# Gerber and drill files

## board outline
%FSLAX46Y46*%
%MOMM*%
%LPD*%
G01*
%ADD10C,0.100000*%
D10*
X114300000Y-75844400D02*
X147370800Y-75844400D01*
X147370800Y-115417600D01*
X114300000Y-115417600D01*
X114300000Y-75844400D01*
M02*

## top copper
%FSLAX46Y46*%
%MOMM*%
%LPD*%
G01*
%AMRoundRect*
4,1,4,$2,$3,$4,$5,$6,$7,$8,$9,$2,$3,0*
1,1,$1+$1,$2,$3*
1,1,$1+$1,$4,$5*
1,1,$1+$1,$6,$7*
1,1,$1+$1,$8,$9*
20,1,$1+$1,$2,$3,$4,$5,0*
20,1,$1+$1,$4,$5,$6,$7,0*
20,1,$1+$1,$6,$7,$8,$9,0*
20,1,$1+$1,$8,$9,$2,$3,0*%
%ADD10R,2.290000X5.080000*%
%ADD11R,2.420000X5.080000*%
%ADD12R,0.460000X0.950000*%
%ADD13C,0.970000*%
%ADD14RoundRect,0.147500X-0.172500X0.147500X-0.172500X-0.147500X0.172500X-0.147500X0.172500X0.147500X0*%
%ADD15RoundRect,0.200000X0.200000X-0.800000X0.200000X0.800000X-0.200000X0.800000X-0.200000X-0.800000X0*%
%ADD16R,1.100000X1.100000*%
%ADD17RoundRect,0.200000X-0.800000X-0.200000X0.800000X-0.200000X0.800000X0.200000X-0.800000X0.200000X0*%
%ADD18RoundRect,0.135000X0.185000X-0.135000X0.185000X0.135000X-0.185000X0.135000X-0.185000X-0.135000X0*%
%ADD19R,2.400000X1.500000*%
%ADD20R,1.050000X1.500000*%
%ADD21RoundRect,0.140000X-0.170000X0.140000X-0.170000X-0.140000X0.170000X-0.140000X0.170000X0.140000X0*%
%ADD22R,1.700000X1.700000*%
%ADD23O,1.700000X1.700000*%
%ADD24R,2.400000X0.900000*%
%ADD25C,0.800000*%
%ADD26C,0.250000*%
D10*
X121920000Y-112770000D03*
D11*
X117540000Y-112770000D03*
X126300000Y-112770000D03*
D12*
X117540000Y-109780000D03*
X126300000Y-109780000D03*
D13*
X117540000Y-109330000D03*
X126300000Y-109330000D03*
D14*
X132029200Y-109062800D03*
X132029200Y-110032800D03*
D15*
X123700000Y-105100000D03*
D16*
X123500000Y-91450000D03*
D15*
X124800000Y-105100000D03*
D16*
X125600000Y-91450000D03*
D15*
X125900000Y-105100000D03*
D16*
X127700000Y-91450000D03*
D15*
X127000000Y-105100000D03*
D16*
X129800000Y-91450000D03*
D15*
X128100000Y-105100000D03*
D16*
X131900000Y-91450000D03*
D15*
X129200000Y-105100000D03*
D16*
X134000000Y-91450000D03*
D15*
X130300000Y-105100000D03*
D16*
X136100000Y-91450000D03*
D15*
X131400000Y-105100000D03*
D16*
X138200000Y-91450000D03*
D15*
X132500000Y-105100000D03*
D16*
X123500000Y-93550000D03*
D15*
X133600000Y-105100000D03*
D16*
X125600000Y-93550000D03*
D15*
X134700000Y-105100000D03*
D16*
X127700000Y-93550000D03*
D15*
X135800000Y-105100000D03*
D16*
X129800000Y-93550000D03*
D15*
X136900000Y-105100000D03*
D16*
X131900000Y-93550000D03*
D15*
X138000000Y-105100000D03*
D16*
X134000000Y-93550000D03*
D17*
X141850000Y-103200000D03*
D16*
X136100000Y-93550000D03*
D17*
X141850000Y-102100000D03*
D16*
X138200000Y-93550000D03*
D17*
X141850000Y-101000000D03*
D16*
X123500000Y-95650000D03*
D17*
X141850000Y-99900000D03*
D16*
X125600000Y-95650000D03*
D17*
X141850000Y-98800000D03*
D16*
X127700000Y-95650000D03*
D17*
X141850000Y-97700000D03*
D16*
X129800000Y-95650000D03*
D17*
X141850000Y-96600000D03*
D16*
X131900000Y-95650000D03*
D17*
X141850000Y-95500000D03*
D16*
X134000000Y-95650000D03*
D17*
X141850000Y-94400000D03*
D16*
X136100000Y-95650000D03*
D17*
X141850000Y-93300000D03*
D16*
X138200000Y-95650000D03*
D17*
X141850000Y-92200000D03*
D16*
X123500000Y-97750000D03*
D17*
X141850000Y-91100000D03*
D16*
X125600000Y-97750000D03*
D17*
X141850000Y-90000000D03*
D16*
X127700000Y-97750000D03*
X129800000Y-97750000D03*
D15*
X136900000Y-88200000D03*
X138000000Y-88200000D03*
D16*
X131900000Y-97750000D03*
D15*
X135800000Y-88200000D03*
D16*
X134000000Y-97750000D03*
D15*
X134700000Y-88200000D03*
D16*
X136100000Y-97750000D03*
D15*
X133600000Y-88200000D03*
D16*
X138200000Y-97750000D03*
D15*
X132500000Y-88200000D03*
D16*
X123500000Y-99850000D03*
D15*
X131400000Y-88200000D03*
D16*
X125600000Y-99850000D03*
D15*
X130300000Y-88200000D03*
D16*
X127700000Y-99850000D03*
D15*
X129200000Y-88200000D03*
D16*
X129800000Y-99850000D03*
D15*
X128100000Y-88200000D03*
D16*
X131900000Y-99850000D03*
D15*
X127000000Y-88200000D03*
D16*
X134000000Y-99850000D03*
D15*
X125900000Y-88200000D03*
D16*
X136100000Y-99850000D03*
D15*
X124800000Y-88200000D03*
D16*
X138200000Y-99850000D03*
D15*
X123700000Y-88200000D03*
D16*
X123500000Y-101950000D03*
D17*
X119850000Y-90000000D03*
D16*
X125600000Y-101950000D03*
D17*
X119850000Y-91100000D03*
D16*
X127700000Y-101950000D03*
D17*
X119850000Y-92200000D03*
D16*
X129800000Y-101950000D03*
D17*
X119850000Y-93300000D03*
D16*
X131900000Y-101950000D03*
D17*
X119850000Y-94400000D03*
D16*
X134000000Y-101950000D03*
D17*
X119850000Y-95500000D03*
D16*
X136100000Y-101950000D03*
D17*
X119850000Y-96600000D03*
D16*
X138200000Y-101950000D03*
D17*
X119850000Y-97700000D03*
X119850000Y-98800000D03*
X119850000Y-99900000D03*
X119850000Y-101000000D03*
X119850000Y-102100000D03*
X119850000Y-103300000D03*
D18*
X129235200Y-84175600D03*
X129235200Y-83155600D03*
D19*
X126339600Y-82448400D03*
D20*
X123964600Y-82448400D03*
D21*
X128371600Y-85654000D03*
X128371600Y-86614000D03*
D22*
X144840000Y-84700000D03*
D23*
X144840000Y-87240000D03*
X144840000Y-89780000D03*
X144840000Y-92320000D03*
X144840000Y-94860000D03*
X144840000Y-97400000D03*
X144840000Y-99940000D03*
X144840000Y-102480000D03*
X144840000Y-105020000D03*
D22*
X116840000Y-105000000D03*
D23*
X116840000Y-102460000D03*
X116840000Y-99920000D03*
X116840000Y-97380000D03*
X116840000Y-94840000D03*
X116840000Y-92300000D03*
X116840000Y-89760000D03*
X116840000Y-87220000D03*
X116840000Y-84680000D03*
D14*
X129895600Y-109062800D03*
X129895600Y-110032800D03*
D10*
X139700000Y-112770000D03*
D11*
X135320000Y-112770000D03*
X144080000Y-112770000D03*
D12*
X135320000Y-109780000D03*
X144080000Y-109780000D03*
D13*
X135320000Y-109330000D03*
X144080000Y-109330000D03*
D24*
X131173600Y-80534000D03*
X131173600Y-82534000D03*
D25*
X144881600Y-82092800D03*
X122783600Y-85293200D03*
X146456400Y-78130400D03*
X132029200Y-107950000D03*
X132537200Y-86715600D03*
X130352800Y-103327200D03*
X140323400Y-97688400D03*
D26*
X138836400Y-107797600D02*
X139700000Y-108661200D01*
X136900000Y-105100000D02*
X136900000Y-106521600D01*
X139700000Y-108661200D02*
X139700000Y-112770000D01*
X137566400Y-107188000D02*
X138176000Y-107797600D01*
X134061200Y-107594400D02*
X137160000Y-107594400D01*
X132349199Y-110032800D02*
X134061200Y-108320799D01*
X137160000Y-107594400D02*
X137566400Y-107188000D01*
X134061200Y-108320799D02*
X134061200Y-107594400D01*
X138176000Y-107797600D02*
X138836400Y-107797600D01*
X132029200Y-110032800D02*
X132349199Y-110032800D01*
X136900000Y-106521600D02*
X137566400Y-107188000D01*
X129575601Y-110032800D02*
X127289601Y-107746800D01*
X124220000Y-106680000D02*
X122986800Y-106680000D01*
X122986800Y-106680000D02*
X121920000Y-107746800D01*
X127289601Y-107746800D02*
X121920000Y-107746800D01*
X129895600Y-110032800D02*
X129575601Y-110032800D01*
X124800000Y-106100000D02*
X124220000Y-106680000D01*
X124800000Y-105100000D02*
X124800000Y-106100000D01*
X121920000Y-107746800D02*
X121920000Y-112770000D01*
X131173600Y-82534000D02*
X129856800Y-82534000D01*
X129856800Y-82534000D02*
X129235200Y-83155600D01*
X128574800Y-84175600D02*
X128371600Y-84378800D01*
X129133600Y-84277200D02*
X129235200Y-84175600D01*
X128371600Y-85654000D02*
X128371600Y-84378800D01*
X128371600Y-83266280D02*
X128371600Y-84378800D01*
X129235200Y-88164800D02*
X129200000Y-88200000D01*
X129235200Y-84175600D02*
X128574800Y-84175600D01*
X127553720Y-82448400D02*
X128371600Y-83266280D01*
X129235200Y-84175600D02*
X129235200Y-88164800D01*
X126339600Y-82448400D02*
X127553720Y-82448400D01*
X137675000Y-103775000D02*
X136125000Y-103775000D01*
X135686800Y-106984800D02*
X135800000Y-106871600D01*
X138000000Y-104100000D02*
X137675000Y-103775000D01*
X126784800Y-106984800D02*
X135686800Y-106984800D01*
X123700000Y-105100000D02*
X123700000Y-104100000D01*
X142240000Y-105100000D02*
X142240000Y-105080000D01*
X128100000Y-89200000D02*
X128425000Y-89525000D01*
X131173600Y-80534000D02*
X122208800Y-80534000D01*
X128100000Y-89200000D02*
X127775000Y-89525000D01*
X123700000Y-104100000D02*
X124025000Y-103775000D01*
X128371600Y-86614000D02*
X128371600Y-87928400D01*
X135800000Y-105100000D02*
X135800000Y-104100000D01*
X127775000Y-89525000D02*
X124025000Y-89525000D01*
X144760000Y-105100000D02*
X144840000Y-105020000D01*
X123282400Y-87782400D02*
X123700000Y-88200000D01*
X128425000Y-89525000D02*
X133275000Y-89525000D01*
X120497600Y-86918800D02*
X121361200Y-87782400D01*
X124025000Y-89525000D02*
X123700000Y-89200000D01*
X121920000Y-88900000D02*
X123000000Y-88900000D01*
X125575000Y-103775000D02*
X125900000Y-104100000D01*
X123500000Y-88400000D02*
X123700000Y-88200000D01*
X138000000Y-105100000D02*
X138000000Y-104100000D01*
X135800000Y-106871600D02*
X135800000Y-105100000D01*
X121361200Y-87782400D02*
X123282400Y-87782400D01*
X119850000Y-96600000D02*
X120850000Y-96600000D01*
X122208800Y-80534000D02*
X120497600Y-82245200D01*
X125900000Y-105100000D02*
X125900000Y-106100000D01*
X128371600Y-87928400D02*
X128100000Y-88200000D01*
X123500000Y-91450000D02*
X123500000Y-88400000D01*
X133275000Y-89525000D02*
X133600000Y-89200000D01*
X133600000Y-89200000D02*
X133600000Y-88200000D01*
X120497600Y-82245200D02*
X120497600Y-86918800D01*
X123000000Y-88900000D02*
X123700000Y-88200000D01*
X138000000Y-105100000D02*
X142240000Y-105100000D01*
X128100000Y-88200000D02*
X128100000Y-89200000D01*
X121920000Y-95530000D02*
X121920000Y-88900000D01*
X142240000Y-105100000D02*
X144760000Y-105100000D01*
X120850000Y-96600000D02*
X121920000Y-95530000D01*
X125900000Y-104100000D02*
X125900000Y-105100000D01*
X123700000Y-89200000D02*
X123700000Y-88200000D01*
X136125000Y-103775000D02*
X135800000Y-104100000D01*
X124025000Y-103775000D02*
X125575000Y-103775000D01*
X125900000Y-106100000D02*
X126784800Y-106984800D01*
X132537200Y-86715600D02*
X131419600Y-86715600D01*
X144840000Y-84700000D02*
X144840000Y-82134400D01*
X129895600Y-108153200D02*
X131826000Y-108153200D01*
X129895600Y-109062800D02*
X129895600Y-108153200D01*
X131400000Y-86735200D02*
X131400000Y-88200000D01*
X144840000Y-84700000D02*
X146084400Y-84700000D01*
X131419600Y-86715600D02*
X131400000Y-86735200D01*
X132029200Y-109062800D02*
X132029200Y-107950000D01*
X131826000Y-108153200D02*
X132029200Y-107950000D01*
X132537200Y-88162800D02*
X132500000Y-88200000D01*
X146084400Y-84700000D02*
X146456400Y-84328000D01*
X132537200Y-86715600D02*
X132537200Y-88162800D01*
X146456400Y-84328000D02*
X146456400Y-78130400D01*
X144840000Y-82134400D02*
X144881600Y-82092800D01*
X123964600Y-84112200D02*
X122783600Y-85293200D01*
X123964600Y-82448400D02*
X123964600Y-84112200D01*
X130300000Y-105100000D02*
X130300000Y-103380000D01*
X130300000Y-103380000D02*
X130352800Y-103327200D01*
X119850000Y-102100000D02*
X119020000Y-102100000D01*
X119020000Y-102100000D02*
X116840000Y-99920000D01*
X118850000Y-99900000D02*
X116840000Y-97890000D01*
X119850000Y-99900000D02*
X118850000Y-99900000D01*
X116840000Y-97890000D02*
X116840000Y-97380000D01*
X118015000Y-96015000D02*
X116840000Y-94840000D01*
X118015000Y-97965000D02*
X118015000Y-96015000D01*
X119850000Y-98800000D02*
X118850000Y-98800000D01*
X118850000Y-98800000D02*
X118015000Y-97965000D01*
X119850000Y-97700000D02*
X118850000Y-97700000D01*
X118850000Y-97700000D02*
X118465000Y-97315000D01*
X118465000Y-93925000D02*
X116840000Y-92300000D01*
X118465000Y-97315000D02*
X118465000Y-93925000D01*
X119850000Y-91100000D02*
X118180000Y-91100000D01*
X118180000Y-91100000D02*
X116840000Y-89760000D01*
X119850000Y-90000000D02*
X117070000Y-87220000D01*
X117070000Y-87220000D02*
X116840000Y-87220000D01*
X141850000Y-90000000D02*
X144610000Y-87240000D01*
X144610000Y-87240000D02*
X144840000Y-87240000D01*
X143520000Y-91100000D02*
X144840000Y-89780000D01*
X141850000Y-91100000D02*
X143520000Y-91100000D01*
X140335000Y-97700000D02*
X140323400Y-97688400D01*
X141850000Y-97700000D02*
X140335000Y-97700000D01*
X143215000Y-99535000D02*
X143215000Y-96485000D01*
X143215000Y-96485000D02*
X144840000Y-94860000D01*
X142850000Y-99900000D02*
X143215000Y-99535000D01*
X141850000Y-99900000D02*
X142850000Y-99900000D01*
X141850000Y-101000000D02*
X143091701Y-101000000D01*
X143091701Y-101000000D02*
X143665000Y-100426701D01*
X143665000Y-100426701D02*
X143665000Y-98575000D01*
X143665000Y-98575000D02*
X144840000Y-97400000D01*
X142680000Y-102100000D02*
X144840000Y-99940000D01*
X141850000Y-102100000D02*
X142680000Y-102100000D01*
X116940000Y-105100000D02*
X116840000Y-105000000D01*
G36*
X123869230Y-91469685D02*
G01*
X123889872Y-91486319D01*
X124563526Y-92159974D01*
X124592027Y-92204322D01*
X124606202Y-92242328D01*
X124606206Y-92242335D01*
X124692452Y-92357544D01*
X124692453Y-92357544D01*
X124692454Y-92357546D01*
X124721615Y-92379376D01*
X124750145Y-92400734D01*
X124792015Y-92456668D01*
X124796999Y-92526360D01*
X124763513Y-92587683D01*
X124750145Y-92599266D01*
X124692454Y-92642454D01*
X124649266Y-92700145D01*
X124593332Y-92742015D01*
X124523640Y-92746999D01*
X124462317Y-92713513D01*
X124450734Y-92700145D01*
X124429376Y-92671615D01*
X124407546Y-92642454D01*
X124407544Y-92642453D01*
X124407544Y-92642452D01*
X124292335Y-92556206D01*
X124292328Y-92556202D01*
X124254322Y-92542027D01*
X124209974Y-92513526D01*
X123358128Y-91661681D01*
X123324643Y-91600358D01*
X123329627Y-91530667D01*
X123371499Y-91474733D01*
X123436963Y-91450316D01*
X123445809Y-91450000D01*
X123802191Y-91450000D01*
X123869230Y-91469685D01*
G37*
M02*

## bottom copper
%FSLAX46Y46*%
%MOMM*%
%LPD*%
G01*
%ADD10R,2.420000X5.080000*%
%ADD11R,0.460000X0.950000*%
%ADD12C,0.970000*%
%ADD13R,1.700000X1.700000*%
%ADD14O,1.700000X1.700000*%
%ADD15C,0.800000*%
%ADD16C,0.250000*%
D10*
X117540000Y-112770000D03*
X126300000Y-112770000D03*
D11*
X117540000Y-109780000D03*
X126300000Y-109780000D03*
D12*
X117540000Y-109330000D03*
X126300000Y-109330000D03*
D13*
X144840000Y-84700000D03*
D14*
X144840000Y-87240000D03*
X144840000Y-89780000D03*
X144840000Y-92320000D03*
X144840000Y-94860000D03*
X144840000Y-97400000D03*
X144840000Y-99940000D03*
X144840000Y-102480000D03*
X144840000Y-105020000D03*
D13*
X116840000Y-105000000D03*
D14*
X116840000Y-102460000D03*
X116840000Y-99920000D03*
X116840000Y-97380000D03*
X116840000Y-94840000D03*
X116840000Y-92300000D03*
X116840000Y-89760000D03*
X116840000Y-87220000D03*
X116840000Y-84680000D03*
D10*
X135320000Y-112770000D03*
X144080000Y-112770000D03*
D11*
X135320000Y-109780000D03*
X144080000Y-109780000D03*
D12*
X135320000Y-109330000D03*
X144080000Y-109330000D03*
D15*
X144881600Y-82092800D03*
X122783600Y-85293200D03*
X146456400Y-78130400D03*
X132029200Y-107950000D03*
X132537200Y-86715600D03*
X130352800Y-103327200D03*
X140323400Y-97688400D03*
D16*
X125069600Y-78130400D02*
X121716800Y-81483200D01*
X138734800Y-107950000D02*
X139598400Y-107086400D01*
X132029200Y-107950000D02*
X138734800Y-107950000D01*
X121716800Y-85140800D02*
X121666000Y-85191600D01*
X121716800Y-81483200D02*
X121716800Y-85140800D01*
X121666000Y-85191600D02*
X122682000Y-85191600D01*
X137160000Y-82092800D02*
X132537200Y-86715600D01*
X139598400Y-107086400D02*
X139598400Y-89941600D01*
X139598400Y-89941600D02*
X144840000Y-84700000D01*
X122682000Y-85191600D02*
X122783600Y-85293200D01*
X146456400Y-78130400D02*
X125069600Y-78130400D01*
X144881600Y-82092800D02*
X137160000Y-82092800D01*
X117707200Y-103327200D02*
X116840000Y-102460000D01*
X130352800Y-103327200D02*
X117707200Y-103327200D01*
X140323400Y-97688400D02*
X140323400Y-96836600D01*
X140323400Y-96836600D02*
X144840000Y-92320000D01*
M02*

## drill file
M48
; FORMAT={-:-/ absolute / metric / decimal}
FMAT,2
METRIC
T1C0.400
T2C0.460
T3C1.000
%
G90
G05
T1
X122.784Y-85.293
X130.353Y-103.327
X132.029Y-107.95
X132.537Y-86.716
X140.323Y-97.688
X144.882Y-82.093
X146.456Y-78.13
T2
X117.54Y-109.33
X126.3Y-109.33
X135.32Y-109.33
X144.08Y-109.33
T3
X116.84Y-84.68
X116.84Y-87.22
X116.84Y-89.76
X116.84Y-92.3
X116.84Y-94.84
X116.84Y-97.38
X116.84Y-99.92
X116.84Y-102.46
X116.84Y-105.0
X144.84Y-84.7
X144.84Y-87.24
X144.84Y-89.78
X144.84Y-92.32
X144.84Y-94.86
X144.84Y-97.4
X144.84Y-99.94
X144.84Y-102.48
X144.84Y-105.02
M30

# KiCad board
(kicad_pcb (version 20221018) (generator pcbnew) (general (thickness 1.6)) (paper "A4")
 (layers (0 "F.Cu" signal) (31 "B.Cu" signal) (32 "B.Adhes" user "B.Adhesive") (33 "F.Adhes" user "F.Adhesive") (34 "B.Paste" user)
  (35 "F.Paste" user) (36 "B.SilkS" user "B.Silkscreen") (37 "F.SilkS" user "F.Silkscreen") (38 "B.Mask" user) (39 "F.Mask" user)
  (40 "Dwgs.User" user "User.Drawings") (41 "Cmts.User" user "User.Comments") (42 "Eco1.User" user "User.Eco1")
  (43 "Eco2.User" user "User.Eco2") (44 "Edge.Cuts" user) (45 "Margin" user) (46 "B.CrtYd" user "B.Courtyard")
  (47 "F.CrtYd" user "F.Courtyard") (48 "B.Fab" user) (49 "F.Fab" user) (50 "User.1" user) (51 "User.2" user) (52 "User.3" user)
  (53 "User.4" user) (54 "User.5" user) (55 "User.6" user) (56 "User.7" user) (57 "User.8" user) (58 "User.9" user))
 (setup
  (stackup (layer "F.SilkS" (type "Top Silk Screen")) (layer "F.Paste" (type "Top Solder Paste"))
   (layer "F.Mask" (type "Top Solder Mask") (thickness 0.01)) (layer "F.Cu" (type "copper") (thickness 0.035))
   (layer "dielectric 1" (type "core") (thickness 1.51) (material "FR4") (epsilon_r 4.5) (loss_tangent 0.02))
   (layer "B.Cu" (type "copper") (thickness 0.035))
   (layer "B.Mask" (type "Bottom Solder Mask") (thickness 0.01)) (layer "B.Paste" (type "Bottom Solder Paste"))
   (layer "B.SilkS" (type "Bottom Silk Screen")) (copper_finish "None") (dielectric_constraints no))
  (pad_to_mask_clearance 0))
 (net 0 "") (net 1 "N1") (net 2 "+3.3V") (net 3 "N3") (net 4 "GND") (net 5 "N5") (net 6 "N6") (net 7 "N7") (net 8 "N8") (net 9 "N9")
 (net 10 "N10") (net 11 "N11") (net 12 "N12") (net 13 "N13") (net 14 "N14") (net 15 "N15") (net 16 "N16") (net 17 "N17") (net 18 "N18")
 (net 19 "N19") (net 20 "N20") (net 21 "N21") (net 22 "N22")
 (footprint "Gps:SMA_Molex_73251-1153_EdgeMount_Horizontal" (layer "F.Cu") (at 121.92 111.05 90)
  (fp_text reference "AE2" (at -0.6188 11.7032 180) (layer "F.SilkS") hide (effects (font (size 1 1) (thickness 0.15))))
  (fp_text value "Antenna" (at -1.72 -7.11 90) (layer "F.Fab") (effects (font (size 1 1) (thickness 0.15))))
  (pad "1" smd rect (at -1.72 0 90) (size 5.08 2.29) (layers "F.Cu" "F.Paste" "F.Mask") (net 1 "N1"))
  (pad "2" smd rect (at -1.72 -4.38 90) (size 5.08 2.42) (layers "F.Cu" "F.Paste" "F.Mask"))
  (pad "2" smd rect (at -1.72 -4.38 90) (size 5.08 2.42) (layers "B.Cu" "B.Paste" "B.Mask"))
  (pad "2" smd rect (at -1.72 4.38 90) (size 5.08 2.42) (layers "F.Cu" "F.Paste" "F.Mask"))
  (pad "2" smd rect (at -1.72 4.38 90) (size 5.08 2.42) (layers "B.Cu" "B.Paste" "B.Mask"))
  (pad "2" smd rect (at 1.27 -4.38 90) (size 0.95 0.46) (layers "F.Cu"))
  (pad "2" smd rect (at 1.27 -4.38 90) (size 0.95 0.46) (layers "B.Cu"))
  (pad "2" smd rect (at 1.27 4.38 90) (size 0.95 0.46) (layers "F.Cu"))
  (pad "2" smd rect (at 1.27 4.38 90) (size 0.95 0.46) (layers "B.Cu"))
  (pad "2" thru_hole circle (at 1.72 -4.38 90) (size 0.97 0.97) (drill 0.46) (layers "*.Cu"))
  (pad "2" thru_hole circle (at 1.72 4.38 90) (size 0.97 0.97) (drill 0.46) (layers "*.Cu")))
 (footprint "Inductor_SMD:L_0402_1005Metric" (layer "F.Cu") (at 132.0292 109.5478 -90)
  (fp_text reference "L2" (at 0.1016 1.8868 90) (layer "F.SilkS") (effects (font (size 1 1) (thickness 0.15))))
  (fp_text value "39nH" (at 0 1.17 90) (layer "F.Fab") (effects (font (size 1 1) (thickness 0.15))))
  (pad "1" smd roundrect (at -0.485 0 270) (size 0.59 0.64) (layers "F.Cu" "F.Paste" "F.Mask") (roundrect_rratio 0.25) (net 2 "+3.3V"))
  (pad "2" smd roundrect (at 0.485 0 270) (size 0.59 0.64) (layers "F.Cu" "F.Paste" "F.Mask") (roundrect_rratio 0.25) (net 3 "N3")))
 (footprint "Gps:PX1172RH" (layer "F.Cu") (at 119.85 90)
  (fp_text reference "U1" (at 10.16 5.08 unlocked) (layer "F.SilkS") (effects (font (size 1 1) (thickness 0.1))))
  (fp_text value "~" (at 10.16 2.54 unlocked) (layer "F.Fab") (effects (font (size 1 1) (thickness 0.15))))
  (pad "1" smd roundrect (at 3.85 15.1 90) (size 2 0.8) (layers "F.Cu" "F.Paste" "F.Mask") (roundrect_rratio 0.25) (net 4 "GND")
   (thermal_bridge_angle 45))
  (pad "1$" smd rect (at 3.65 1.45) (size 1.1 1.1) (layers "F.Cu" "F.Paste" "F.Mask") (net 4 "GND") (thermal_bridge_angle 45))
  (pad "2" smd roundrect (at 4.95 15.1 90) (size 2 0.8) (layers "F.Cu" "F.Paste" "F.Mask") (roundrect_rratio 0.25) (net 1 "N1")
   (thermal_bridge_angle 45))
  (pad "2$" smd rect (at 5.75 1.45) (size 1.1 1.1) (layers "F.Cu" "F.Paste" "F.Mask") (thermal_bridge_angle 45))
  (pad "3" smd roundrect (at 6.05 15.1 90) (size 2 0.8) (layers "F.Cu" "F.Paste" "F.Mask") (roundrect_rratio 0.25) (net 4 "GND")
   (thermal_bridge_angle 45))
  (pad "3$" smd rect (at 7.85 1.45) (size 1.1 1.1) (layers "F.Cu" "F.Paste" "F.Mask") (thermal_bridge_angle 45))
  (pad "4" smd roundrect (at 7.15 15.1 90) (size 2 0.8) (layers "F.Cu" "F.Paste" "F.Mask") (roundrect_rratio 0.25) (thermal_bridge_angle 45))
  (pad "4$" smd rect (at 9.95 1.45) (size 1.1 1.1) (layers "F.Cu" "F.Paste" "F.Mask") (thermal_bridge_angle 45))
  (pad "5" smd roundrect (at 8.25 15.1 90) (size 2 0.8) (layers "F.Cu" "F.Paste" "F.Mask") (roundrect_rratio 0.25) (thermal_bridge_angle 45))
  (pad "5$" smd rect (at 12.05 1.45) (size 1.1 1.1) (layers "F.Cu" "F.Paste" "F.Mask") (thermal_bridge_angle 45))
  (pad "6" smd roundrect (at 9.35 15.1 90) (size 2 0.8) (layers "F.Cu" "F.Paste" "F.Mask") (roundrect_rratio 0.25) (thermal_bridge_angle 45))
  (pad "6$" smd rect (at 14.15 1.45) (size 1.1 1.1) (layers "F.Cu" "F.Paste" "F.Mask") (thermal_bridge_angle 45))
  (pad "7" smd roundrect (at 10.45 15.1 90) (size 2 0.8) (layers "F.Cu" "F.Paste" "F.Mask") (roundrect_rratio 0.25) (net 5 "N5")
   (thermal_bridge_angle 45))
  (pad "7$" smd rect (at 16.25 1.45) (size 1.1 1.1) (layers "F.Cu" "F.Paste" "F.Mask") (thermal_bridge_angle 45))
  (pad "8" smd roundrect (at 11.55 15.1 90) (size 2 0.8) (layers "F.Cu" "F.Paste" "F.Mask") (roundrect_rratio 0.25)
   (thermal_bridge_angle 45))
  (pad "8$" smd rect (at 18.35 1.45) (size 1.1 1.1) (layers "F.Cu" "F.Paste" "F.Mask") (thermal_bridge_angle 45))
  (pad "9" smd roundrect (at 12.65 15.1 90) (size 2 0.8) (layers "F.Cu" "F.Paste" "F.Mask") (roundrect_rratio 0.25)
   (thermal_bridge_angle 45))
  (pad "9$" smd rect (at 3.65 3.55) (size 1.1 1.1) (layers "F.Cu" "F.Paste" "F.Mask") (thermal_bridge_angle 45))
  (pad "10" smd roundrect (at 13.75 15.1 90) (size 2 0.8) (layers "F.Cu" "F.Paste" "F.Mask") (roundrect_rratio 0.25)
   (thermal_bridge_angle 45))
  (pad "10$" smd rect (at 5.75 3.55) (size 1.1 1.1) (layers "F.Cu" "F.Paste" "F.Mask") (thermal_bridge_angle 45))
  (pad "11" smd roundrect (at 14.85 15.1 90) (size 2 0.8) (layers "F.Cu" "F.Paste" "F.Mask") (roundrect_rratio 0.25)
   (thermal_bridge_angle 45))
  (pad "11$" smd rect (at 7.85 3.55) (size 1.1 1.1) (layers "F.Cu" "F.Paste" "F.Mask") (thermal_bridge_angle 45))
  (pad "12" smd roundrect (at 15.95 15.1 90) (size 2 0.8) (layers "F.Cu" "F.Paste" "F.Mask") (roundrect_rratio 0.25) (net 4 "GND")
   (thermal_bridge_angle 45))
  (pad "12$" smd rect (at 9.95 3.55) (size 1.1 1.1) (layers "F.Cu" "F.Paste" "F.Mask") (thermal_bridge_angle 45))
  (pad "13" smd roundrect (at 17.05 15.1 90) (size 2 0.8) (layers "F.Cu" "F.Paste" "F.Mask") (roundrect_rratio 0.25) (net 3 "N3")
   (thermal_bridge_angle 45))
  (pad "13$" smd rect (at 12.05 3.55) (size 1.1 1.1) (layers "F.Cu" "F.Paste" "F.Mask") (thermal_bridge_angle 45))
  (pad "14" smd roundrect (at 18.15 15.1 90) (size 2 0.8) (layers "F.Cu" "F.Paste" "F.Mask") (roundrect_rratio 0.25) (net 4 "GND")
   (thermal_bridge_angle 45))
  (pad "14$" smd rect (at 14.15 3.55) (size 1.1 1.1) (layers "F.Cu" "F.Paste" "F.Mask") (thermal_bridge_angle 45))
  (pad "15" smd roundrect (at 22 13.2) (size 2 0.8) (layers "F.Cu" "F.Paste" "F.Mask") (roundrect_rratio 0.25) (thermal_bridge_angle 45))
  (pad "15$" smd rect (at 16.25 3.55) (size 1.1 1.1) (layers "F.Cu" "F.Paste" "F.Mask") (thermal_bridge_angle 45))
  (pad "16" smd roundrect (at 22 12.1) (size 2 0.8) (layers "F.Cu" "F.Paste" "F.Mask") (roundrect_rratio 0.25) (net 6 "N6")
   (thermal_bridge_angle 45))
  (pad "16$" smd rect (at 18.35 3.55) (size 1.1 1.1) (layers "F.Cu" "F.Paste" "F.Mask") (thermal_bridge_angle 45))
  (pad "17" smd roundrect (at 22 11) (size 2 0.8) (layers "F.Cu" "F.Paste" "F.Mask") (roundrect_rratio 0.25) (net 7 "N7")
   (thermal_bridge_angle 45))
  (pad "17$" smd rect (at 3.65 5.65) (size 1.1 1.1) (layers "F.Cu" "F.Paste" "F.Mask") (thermal_bridge_angle 45))
  (pad "18" smd roundrect (at 22 9.9) (size 2 0.8) (layers "F.Cu" "F.Paste" "F.Mask") (roundrect_rratio 0.25) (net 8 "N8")
   (thermal_bridge_angle 45))
  (pad "18$" smd rect (at 5.75 5.65) (size 1.1 1.1) (layers "F.Cu" "F.Paste" "F.Mask") (thermal_bridge_angle 45))
  (pad "19" smd roundrect (at 22 8.8) (size 2 0.8) (layers "F.Cu" "F.Paste" "F.Mask") (roundrect_rratio 0.25) (thermal_bridge_angle 45))
  (pad "19$" smd rect (at 7.85 5.65) (size 1.1 1.1) (layers "F.Cu" "F.Paste" "F.Mask") (thermal_bridge_angle 45))
  (pad "20" smd roundrect (at 22 7.7) (size 2 0.8) (layers "F.Cu" "F.Paste" "F.Mask") (roundrect_rratio 0.25) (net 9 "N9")
   (thermal_bridge_angle 45))
  (pad "20$" smd rect (at 9.95 5.65) (size 1.1 1.1) (layers "F.Cu" "F.Paste" "F.Mask") (thermal_bridge_angle 45))
  (pad "21" smd roundrect (at 22 6.6) (size 2 0.8) (layers "F.Cu" "F.Paste" "F.Mask") (roundrect_rratio 0.25) (thermal_bridge_angle 45))
  (pad "21$" smd rect (at 12.05 5.65) (size 1.1 1.1) (layers "F.Cu" "F.Paste" "F.Mask") (thermal_bridge_angle 45))
  (pad "22" smd roundrect (at 22 5.5) (size 2 0.8) (layers "F.Cu" "F.Paste" "F.Mask") (roundrect_rratio 0.25) (thermal_bridge_angle 45))
  (pad "22$" smd rect (at 14.15 5.65) (size 1.1 1.1) (layers "F.Cu" "F.Paste" "F.Mask") (thermal_bridge_angle 45))
  (pad "23" smd roundrect (at 22 4.4) (size 2 0.8) (layers "F.Cu" "F.Paste" "F.Mask") (roundrect_rratio 0.25) (thermal_bridge_angle 45))
  (pad "23$" smd rect (at 16.25 5.65) (size 1.1 1.1) (layers "F.Cu" "F.Paste" "F.Mask") (thermal_bridge_angle 45))
  (pad "24" smd roundrect (at 22 3.3) (size 2 0.8) (layers "F.Cu" "F.Paste" "F.Mask") (roundrect_rratio 0.25) (thermal_bridge_angle 45))
  (pad "24$" smd rect (at 18.35 5.65) (size 1.1 1.1) (layers "F.Cu" "F.Paste" "F.Mask") (thermal_bridge_angle 45))
  (pad "25" smd roundrect (at 22 2.2) (size 2 0.8) (layers "F.Cu" "F.Mask") (roundrect_rratio 0.25) (thermal_bridge_angle 45))
  (pad "25$" smd rect (at 3.65 7.75) (size 1.1 1.1) (layers "F.Cu" "F.Paste" "F.Mask") (thermal_bridge_angle 45))
  (pad "26" smd roundrect (at 22 1.1) (size 2 0.8) (layers "F.Cu" "F.Paste" "F.Mask") (roundrect_rratio 0.25) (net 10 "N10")
   (thermal_bridge_angle 45))
  (pad "26$" smd rect (at 5.75 7.75) (size 1.1 1.1) (layers "F.Cu" "F.Paste" "F.Mask") (thermal_bridge_angle 45))
  (pad "27" smd roundrect (at 22 0) (size 2 0.8) (layers "F.Cu" "F.Paste" "F.Mask") (roundrect_rratio 0.25) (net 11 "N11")
   (thermal_bridge_angle 45))
  (pad "27$" smd rect (at 7.85 7.75) (size 1.1 1.1) (layers "F.Cu" "F.Paste" "F.Mask") (thermal_bridge_angle 45))
  (pad "28$" smd rect (at 9.95 7.75) (size 1.1 1.1) (layers "F.Cu" "F.Paste" "F.Mask") (thermal_bridge_angle 45))
  (pad "29" smd roundrect (at 17.05 -1.8 90) (size 2 0.8) (layers "F.Cu" "F.Paste" "F.Mask") (roundrect_rratio 0.25)
   (thermal_bridge_angle 45))
  (pad "29" smd roundrect (at 18.15 -1.8 90) (size 2 0.8) (layers "F.Cu" "F.Paste" "F.Mask") (roundrect_rratio 0.25)
   (thermal_bridge_angle 45))
  (pad "29$" smd rect (at 12.05 7.75) (size 1.1 1.1) (layers "F.Cu" "F.Paste" "F.Mask") (thermal_bridge_angle 45))
  (pad "30" smd roundrect (at 15.95 -1.8 90) (size 2 0.8) (layers "F.Cu" "F.Paste" "F.Mask") (roundrect_rratio 0.25)
   (thermal_bridge_angle 45))
  (pad "30$" smd rect (at 14.15 7.75) (size 1.1 1.1) (layers "F.Cu" "F.Paste" "F.Mask") (thermal_bridge_angle 45))
  (pad "31" smd roundrect (at 14.85 -1.8 90) (size 2 0.8) (layers "F.Cu" "F.Paste" "F.Mask") (roundrect_rratio 0.25)
   (thermal_bridge_angle 45))
  (pad "31$" smd rect (at 16.25 7.75) (size 1.1 1.1) (layers "F.Cu" "F.Paste" "F.Mask") (thermal_bridge_angle 45))
  (pad "32" smd roundrect (at 13.75 -1.8 90) (size 2 0.8) (layers "F.Cu" "F.Paste" "F.Mask") (roundrect_rratio 0.25) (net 4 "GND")
   (thermal_bridge_angle 45))
  (pad "32$" smd rect (at 18.35 7.75) (size 1.1 1.1) (layers "F.Cu" "F.Paste" "F.Mask") (thermal_bridge_angle 45))
  (pad "33" smd roundrect (at 12.65 -1.8 90) (size 2 0.8) (layers "F.Cu" "F.Paste" "F.Mask") (roundrect_rratio 0.25) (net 2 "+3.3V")
   (thermal_bridge_angle 45))
  (pad "33$" smd rect (at 3.65 9.85) (size 1.1 1.1) (layers "F.Cu" "F.Paste" "F.Mask") (thermal_bridge_angle 45))
  (pad "34" smd roundrect (at 11.55 -1.8 90) (size 2 0.8) (layers "F.Cu" "F.Paste" "F.Mask") (roundrect_rratio 0.25) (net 2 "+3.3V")
   (thermal_bridge_angle 45))
  (pad "34$" smd rect (at 5.75 9.85) (size 1.1 1.1) (layers "F.Cu" "F.Paste" "F.Mask") (thermal_bridge_angle 45))
  (pad "35" smd roundrect (at 10.45 -1.8 90) (size 2 0.8) (layers "F.Cu" "F.Paste" "F.Mask") (roundrect_rratio 0.25)
   (thermal_bridge_angle 45))
  (pad "35$" smd rect (at 7.85 9.85) (size 1.1 1.1) (layers "F.Cu" "F.Paste" "F.Mask") (thermal_bridge_angle 45))
  (pad "36" smd roundrect (at 9.35 -1.8 90) (size 2 0.8) (layers "F.Cu" "F.Paste" "F.Mask") (roundrect_rratio 0.25) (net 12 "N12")
   (thermal_bridge_angle 45))
  (pad "36$" smd rect (at 9.95 9.85) (size 1.1 1.1) (layers "F.Cu" "F.Paste" "F.Mask") (thermal_bridge_angle 45))
  (pad "37" smd roundrect (at 8.25 -1.8 90) (size 2 0.8) (layers "F.Cu" "F.Paste" "F.Mask") (roundrect_rratio 0.25) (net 4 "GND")
   (thermal_bridge_angle 45))
  (pad "37$" smd rect (at 12.05 9.85) (size 1.1 1.1) (layers "F.Cu" "F.Paste" "F.Mask") (thermal_bridge_angle 45))
  (pad "38" smd roundrect (at 7.15 -1.8 90) (size 2 0.8) (layers "F.Cu" "F.Paste" "F.Mask") (roundrect_rratio 0.25)
   (thermal_bridge_angle 45))
  (pad "38$" smd rect (at 14.15 9.85) (size 1.1 1.1) (layers "F.Cu" "F.Paste" "F.Mask") (thermal_bridge_angle 45))
  (pad "39" smd roundrect (at 6.05 -1.8 90) (size 2 0.8) (layers "F.Cu" "F.Paste" "F.Mask") (roundrect_rratio 0.25)
   (thermal_bridge_angle 45))
  (pad "39$" smd rect (at 16.25 9.85) (size 1.1 1.1) (layers "F.Cu" "F.Paste" "F.Mask") (thermal_bridge_angle 45))
  (pad "40" smd roundrect (at 4.95 -1.8 90) (size 2 0.8) (layers "F.Cu" "F.Paste" "F.Mask") (roundrect_rratio 0.25)
   (thermal_bridge_angle 45))
  (pad "40$" smd rect (at 18.35 9.85) (size 1.1 1.1) (layers "F.Cu" "F.Paste" "F.Mask") (thermal_bridge_angle 45))
  (pad "41" smd roundrect (at 3.85 -1.8 90) (size 2 0.8) (layers "F.Cu" "F.Paste" "F.Mask") (roundrect_rratio 0.25) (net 4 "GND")
   (thermal_bridge_angle 45))
  (pad "41$" smd rect (at 3.65 11.95) (size 1.1 1.1) (layers "F.Cu" "F.Paste" "F.Mask") (thermal_bridge_angle 45))
  (pad "42" smd roundrect (at 0 0) (size 2 0.8) (layers "F.Cu" "F.Paste" "F.Mask") (roundrect_rratio 0.25) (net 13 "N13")
   (thermal_bridge_angle 45))
  (pad "42$" smd rect (at 5.75 11.95) (size 1.1 1.1) (layers "F.Cu" "F.Paste" "F.Mask") (thermal_bridge_angle 45))
  (pad "43" smd roundrect (at 0 1.1) (size 2 0.8) (layers "F.Cu" "F.Paste" "F.Mask") (roundrect_rratio 0.25) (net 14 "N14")
   (thermal_bridge_angle 45))
  (pad "43$" smd rect (at 7.85 11.95) (size 1.1 1.1) (layers "F.Cu" "F.Paste" "F.Mask") (thermal_bridge_angle 45))
  (pad "44" smd roundrect (at 0 2.2) (size 2 0.8) (layers "F.Cu" "F.Paste" "F.Mask") (roundrect_rratio 0.25) (thermal_bridge_angle 45))
  (pad "44$" smd rect (at 9.95 11.95) (size 1.1 1.1) (layers "F.Cu" "F.Paste" "F.Mask") (thermal_bridge_angle 45))
  (pad "45" smd roundrect (at 0 3.3) (size 2 0.8) (layers "F.Cu" "F.Paste" "F.Mask") (roundrect_rratio 0.25) (thermal_bridge_angle 45))
  (pad "45$" smd rect (at 12.05 11.95) (size 1.1 1.1) (layers "F.Cu" "F.Paste" "F.Mask") (thermal_bridge_angle 45))
  (pad "46" smd roundrect (at 0 4.4) (size 2 0.8) (layers "F.Cu" "F.Paste" "F.Mask") (roundrect_rratio 0.25) (thermal_bridge_angle 45))
  (pad "46$" smd rect (at 14.15 11.95) (size 1.1 1.1) (layers "F.Cu" "F.Paste" "F.Mask") (thermal_bridge_angle 45))
  (pad "47" smd roundrect (at 0 5.5) (size 2 0.8) (layers "F.Cu" "F.Paste" "F.Mask") (roundrect_rratio 0.25) (thermal_bridge_angle 45))
  (pad "47$" smd rect (at 16.25 11.95) (size 1.1 1.1) (layers "F.Cu" "F.Paste" "F.Mask") (thermal_bridge_angle 45))
  (pad "48" smd roundrect (at 0 6.6) (size 2 0.8) (layers "F.Cu" "F.Paste" "F.Mask") (roundrect_rratio 0.25) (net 4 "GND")
   (thermal_bridge_angle 45))
  (pad "48$" smd rect (at 18.35 11.95) (size 1.1 1.1) (layers "F.Cu" "F.Paste" "F.Mask") (thermal_bridge_angle 45))
  (pad "49" smd roundrect (at 0 7.7) (size 2 0.8) (layers "F.Cu" "F.Paste" "F.Mask") (roundrect_rratio 0.25) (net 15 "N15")
   (thermal_bridge_angle 45))
  (pad "50" smd roundrect (at 0 8.8) (size 2 0.8) (layers "F.Cu" "F.Paste" "F.Mask") (roundrect_rratio 0.25) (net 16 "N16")
   (thermal_bridge_angle 45))
  (pad "51" smd roundrect (at 0 9.9) (size 2 0.8) (layers "F.Cu" "F.Paste" "F.Mask") (roundrect_rratio 0.25) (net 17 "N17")
   (thermal_bridge_angle 45))
  (pad "52" smd roundrect (at 0 11) (size 2 0.8) (layers "F.Cu" "F.Paste" "F.Mask") (roundrect_rratio 0.25) (thermal_bridge_angle 45))
  (pad "53" smd roundrect (at 0 12.1) (size 2 0.8) (layers "F.Cu" "F.Paste" "F.Mask") (roundrect_rratio 0.25) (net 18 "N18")
   (thermal_bridge_angle 45))
  (pad "54" smd roundrect (at 0 13.3) (size 2 0.8) (layers "F.Cu" "F.Paste" "F.Mask") (roundrect_rratio 0.25) (thermal_bridge_angle 45)))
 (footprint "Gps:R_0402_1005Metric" (layer "F.Cu") (at 129.2352 83.6656 90)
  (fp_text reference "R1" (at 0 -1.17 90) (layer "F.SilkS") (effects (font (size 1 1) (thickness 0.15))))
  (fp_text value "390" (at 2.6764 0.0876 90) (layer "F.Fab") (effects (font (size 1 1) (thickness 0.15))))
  (pad "1" smd roundrect (at -0.51 0 90) (size 0.54 0.64) (layers "F.Cu" "F.Paste" "F.Mask") (roundrect_rratio 0.25) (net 12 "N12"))
  (pad "2" smd roundrect (at 0.51 0 90) (size 0.54 0.64) (layers "F.Cu" "F.Paste" "F.Mask") (roundrect_rratio 0.25) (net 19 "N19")))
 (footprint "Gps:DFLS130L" (layer "F.Cu") (at 126.3396 82.4484)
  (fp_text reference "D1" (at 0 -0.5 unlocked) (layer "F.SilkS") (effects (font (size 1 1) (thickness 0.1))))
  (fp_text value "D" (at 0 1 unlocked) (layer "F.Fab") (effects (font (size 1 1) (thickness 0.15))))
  (pad "1" smd rect (at 0 0) (size 2.4 1.5) (layers "F.Cu" "F.Paste" "F.Mask" "Dwgs.User") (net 12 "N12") (thermal_bridge_angle 45))
  (pad "2" smd rect (at -2.375 0) (size 1.05 1.5) (layers "F.Cu" "F.Paste" "F.Mask") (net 2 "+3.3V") (thermal_bridge_angle 45)))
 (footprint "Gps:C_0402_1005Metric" (layer "F.Cu") (at 128.3716 86.134 -90)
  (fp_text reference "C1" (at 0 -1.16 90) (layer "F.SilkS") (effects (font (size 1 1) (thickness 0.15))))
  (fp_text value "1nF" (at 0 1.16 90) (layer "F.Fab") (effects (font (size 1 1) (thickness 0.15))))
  (pad "1" smd roundrect (at -0.48 0 270) (size 0.56 0.62) (layers "F.Cu" "F.Paste" "F.Mask") (roundrect_rratio 0.25) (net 12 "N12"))
  (pad "2" smd roundrect (at 0.48 0 270) (size 0.56 0.62) (layers "F.Cu" "F.Paste" "F.Mask") (roundrect_rratio 0.25) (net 4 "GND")))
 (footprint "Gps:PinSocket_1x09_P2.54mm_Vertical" (layer "F.Cu") (at 144.84 84.7)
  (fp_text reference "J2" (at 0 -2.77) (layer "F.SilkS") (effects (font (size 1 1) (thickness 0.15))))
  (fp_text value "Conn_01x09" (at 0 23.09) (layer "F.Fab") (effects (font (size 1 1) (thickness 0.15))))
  (pad "1" thru_hole rect (at 0 0) (size 1.7 1.7) (drill 1) (layers "*.Cu" "*.Mask") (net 2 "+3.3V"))
  (pad "2" thru_hole oval (at 0 2.54) (size 1.7 1.7) (drill 1) (layers "*.Cu" "*.Mask") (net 11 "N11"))
  (pad "3" thru_hole oval (at 0 5.08) (size 1.7 1.7) (drill 1) (layers "*.Cu" "*.Mask") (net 10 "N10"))
  (pad "4" thru_hole oval (at 0 7.62) (size 1.7 1.7) (drill 1) (layers "*.Cu" "*.Mask") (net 9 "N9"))
  (pad "5" thru_hole oval (at 0 10.16) (size 1.7 1.7) (drill 1) (layers "*.Cu" "*.Mask") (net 8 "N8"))
  (pad "6" thru_hole oval (at 0 12.7) (size 1.7 1.7) (drill 1) (layers "*.Cu" "*.Mask") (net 7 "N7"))
  (pad "7" thru_hole oval (at 0 15.24) (size 1.7 1.7) (drill 1) (layers "*.Cu" "*.Mask") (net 6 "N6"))
  (pad "8" thru_hole oval (at 0 17.78) (size 1.7 1.7) (drill 1) (layers "*.Cu" "*.Mask") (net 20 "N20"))
  (pad "9" thru_hole oval (at 0 20.32) (size 1.7 1.7) (drill 1) (layers "*.Cu" "*.Mask") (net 4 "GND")))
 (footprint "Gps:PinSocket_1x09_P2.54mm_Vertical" (layer "F.Cu") (at 116.84 105 180)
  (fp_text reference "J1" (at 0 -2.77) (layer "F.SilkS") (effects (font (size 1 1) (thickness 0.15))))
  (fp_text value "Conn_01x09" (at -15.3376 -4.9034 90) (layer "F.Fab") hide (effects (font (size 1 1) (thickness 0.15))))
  (pad "1" thru_hole rect (at 0 0 180) (size 1.7 1.7) (drill 1) (layers "*.Cu" "*.Mask") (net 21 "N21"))
  (pad "2" thru_hole oval (at 0 2.54 180) (size 1.7 1.7) (drill 1) (layers "*.Cu" "*.Mask") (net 5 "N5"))
  (pad "3" thru_hole oval (at 0 5.08 180) (size 1.7 1.7) (drill 1) (layers "*.Cu" "*.Mask") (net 18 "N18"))
  (pad "4" thru_hole oval (at 0 7.62 180) (size 1.7 1.7) (drill 1) (layers "*.Cu" "*.Mask") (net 17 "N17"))
  (pad "5" thru_hole oval (at 0 10.16 180) (size 1.7 1.7) (drill 1) (layers "*.Cu" "*.Mask") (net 16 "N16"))
  (pad "6" thru_hole oval (at 0 12.7 180) (size 1.7 1.7) (drill 1) (layers "*.Cu" "*.Mask") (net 15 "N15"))
  (pad "7" thru_hole oval (at 0 15.24 180) (size 1.7 1.7) (drill 1) (layers "*.Cu" "*.Mask") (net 14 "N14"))
  (pad "8" thru_hole oval (at 0 17.78 180) (size 1.7 1.7) (drill 1) (layers "*.Cu" "*.Mask") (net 13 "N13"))
  (pad "9" thru_hole oval (at 0 20.32 180) (size 1.7 1.7) (drill 1) (layers "*.Cu" "*.Mask") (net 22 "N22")))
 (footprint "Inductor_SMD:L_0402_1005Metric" (layer "F.Cu") (at 129.8956 109.5478 -90)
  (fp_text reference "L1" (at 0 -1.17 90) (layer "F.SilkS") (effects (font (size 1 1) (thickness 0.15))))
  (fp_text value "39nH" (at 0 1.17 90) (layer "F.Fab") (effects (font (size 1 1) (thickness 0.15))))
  (pad "1" smd roundrect (at -0.485 0 270) (size 0.59 0.64) (layers "F.Cu" "F.Paste" "F.Mask") (roundrect_rratio 0.25) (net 2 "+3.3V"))
  (pad "2" smd roundrect (at 0.485 0 270) (size 0.59 0.64) (layers "F.Cu" "F.Paste" "F.Mask") (roundrect_rratio 0.25) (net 1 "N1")))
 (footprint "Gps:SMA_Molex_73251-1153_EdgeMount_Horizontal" (layer "F.Cu") (at 139.7 111.05 90)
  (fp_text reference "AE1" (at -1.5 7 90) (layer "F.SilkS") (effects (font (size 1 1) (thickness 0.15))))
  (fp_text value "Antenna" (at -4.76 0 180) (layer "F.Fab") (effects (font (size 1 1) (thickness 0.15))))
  (pad "1" smd rect (at -1.72 0 90) (size 5.08 2.29) (layers "F.Cu" "F.Paste" "F.Mask") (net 3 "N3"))
  (pad "2" smd rect (at -1.72 -4.38 90) (size 5.08 2.42) (layers "F.Cu" "F.Paste" "F.Mask"))
  (pad "2" smd rect (at -1.72 -4.38 90) (size 5.08 2.42) (layers "B.Cu" "B.Paste" "B.Mask"))
  (pad "2" smd rect (at -1.72 4.38 90) (size 5.08 2.42) (layers "F.Cu" "F.Paste" "F.Mask"))
  (pad "2" smd rect (at -1.72 4.38 90) (size 5.08 2.42) (layers "B.Cu" "B.Paste" "B.Mask"))
  (pad "2" smd rect (at 1.27 -4.38 90) (size 0.95 0.46) (layers "F.Cu"))
  (pad "2" smd rect (at 1.27 -4.38 90) (size 0.95 0.46) (layers "B.Cu"))
  (pad "2" smd rect (at 1.27 4.38 90) (size 0.95 0.46) (layers "F.Cu"))
  (pad "2" smd rect (at 1.27 4.38 90) (size 0.95 0.46) (layers "B.Cu"))
  (pad "2" thru_hole circle (at 1.72 -4.38 90) (size 0.97 0.97) (drill 0.46) (layers "*.Cu"))
  (pad "2" thru_hole circle (at 1.72 4.38 90) (size 0.97 0.97) (drill 0.46) (layers "*.Cu")))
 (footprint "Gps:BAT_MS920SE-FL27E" (layer "F.Cu") (at 138.0236 81.534 90)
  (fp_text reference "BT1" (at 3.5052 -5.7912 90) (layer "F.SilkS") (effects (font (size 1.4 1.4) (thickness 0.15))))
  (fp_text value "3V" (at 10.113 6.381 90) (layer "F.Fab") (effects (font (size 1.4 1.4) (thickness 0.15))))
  (pad "N" smd rect (at 1 -6.85 180) (size 2.4 0.9) (layers "F.Cu" "F.Paste" "F.Mask") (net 4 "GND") (solder_mask_margin 0.102))
  (pad "P" smd rect (at -1 -6.85 180) (size 2.4 0.9) (layers "F.Cu" "F.Paste" "F.Mask") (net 19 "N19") (solder_mask_margin 0.102)))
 (gr_rect (start 114.3 75.8444) (end 147.3708 115.4176) (stroke (width 0.1) (type default)) (fill none) (layer "Edge.Cuts"))
 (segment (start 138.8364 107.7976) (end 139.7 108.6612) (width 0.25) (layer "F.Cu") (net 3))
 (segment (start 136.9 105.1) (end 136.9 106.5216) (width 0.25) (layer "F.Cu") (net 3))
 (segment (start 139.7 108.6612) (end 139.7 112.77) (width 0.25) (layer "F.Cu") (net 3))
 (segment (start 137.5664 107.188) (end 138.176 107.7976) (width 0.25) (layer "F.Cu") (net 3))
 (segment (start 134.0612 107.5944) (end 137.16 107.5944) (width 0.25) (layer "F.Cu") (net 3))
 (segment (start 132.349199 110.0328) (end 134.0612 108.320799) (width 0.25) (layer "F.Cu") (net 3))
 (segment (start 137.16 107.5944) (end 137.5664 107.188) (width 0.25) (layer "F.Cu") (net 3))
 (segment (start 134.0612 108.320799) (end 134.0612 107.5944) (width 0.25) (layer "F.Cu") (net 3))
 (segment (start 138.176 107.7976) (end 138.8364 107.7976) (width 0.25) (layer "F.Cu") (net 3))
 (segment (start 132.0292 110.0328) (end 132.349199 110.0328) (width 0.25) (layer "F.Cu") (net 3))
 (segment (start 136.9 106.5216) (end 137.5664 107.188) (width 0.25) (layer "F.Cu") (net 3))
 (segment (start 129.575601 110.0328) (end 127.289601 107.7468) (width 0.25) (layer "F.Cu") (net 1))
 (segment (start 124.22 106.68) (end 122.9868 106.68) (width 0.25) (layer "F.Cu") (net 1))
 (segment (start 122.9868 106.68) (end 121.92 107.7468) (width 0.25) (layer "F.Cu") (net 1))
 (segment (start 127.289601 107.7468) (end 121.92 107.7468) (width 0.25) (layer "F.Cu") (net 1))
 (segment (start 129.8956 110.0328) (end 129.575601 110.0328) (width 0.25) (layer "F.Cu") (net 1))
 (segment (start 124.8 106.1) (end 124.22 106.68) (width 0.25) (layer "F.Cu") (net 1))
 (segment (start 124.8 105.1) (end 124.8 106.1) (width 0.25) (layer "F.Cu") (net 1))
 (segment (start 121.92 107.7468) (end 121.92 112.77) (width 0.25) (layer "F.Cu") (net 1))
 (segment (start 131.1736 82.534) (end 129.8568 82.534) (width 0.25) (layer "F.Cu") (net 19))
 (segment (start 129.8568 82.534) (end 129.2352 83.1556) (width 0.25) (layer "F.Cu") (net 19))
 (segment (start 128.5748 84.1756) (end 128.3716 84.3788) (width 0.25) (layer "F.Cu") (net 12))
 (segment (start 129.1336 84.2772) (end 129.2352 84.1756) (width 0.25) (layer "F.Cu") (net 12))
 (segment (start 128.3716 85.654) (end 128.3716 84.3788) (width 0.25) (layer "F.Cu") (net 12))
 (segment (start 128.3716 83.26628) (end 128.3716 84.3788) (width 0.25) (layer "F.Cu") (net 12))
 (segment (start 129.2352 88.1648) (end 129.2 88.2) (width 0.25) (layer "F.Cu") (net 12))
 (segment (start 129.2352 84.1756) (end 128.5748 84.1756) (width 0.25) (layer "F.Cu") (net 12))
 (segment (start 127.55372 82.4484) (end 128.3716 83.26628) (width 0.25) (layer "F.Cu") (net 12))
 (segment (start 129.2352 84.1756) (end 129.2352 88.1648) (width 0.25) (layer "F.Cu") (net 12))
 (segment (start 126.3396 82.4484) (end 127.55372 82.4484) (width 0.25) (layer "F.Cu") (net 12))
 (segment (start 137.675 103.775) (end 136.125 103.775) (width 0.25) (layer "F.Cu") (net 4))
 (segment (start 135.6868 106.9848) (end 135.8 106.8716) (width 0.25) (layer "F.Cu") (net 4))
 (segment (start 138 104.1) (end 137.675 103.775) (width 0.25) (layer "F.Cu") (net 4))
 (segment (start 126.7848 106.9848) (end 135.6868 106.9848) (width 0.25) (layer "F.Cu") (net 4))
 (segment (start 123.7 105.1) (end 123.7 104.1) (width 0.25) (layer "F.Cu") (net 4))
 (segment (start 142.24 105.1) (end 142.24 105.08) (width 0.25) (layer "F.Cu") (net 4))
 (segment (start 128.1 89.2) (end 128.425 89.525) (width 0.25) (layer "F.Cu") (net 4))
 (segment (start 131.1736 80.534) (end 122.2088 80.534) (width 0.25) (layer "F.Cu") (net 4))
 (segment (start 128.1 89.2) (end 127.775 89.525) (width 0.25) (layer "F.Cu") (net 4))
 (segment (start 123.7 104.1) (end 124.025 103.775) (width 0.25) (layer "F.Cu") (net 4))
 (segment (start 128.3716 86.614) (end 128.3716 87.9284) (width 0.25) (layer "F.Cu") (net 4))
 (segment (start 135.8 105.1) (end 135.8 104.1) (width 0.25) (layer "F.Cu") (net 4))
 (segment (start 127.775 89.525) (end 124.025 89.525) (width 0.25) (layer "F.Cu") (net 4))
 (segment (start 144.76 105.1) (end 144.84 105.02) (width 0.25) (layer "F.Cu") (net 4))
 (segment (start 123.2824 87.7824) (end 123.7 88.2) (width 0.25) (layer "F.Cu") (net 4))
 (segment (start 128.425 89.525) (end 133.275 89.525) (width 0.25) (layer "F.Cu") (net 4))
 (segment (start 120.4976 86.9188) (end 121.3612 87.7824) (width 0.25) (layer "F.Cu") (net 4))
 (segment (start 124.025 89.525) (end 123.7 89.2) (width 0.25) (layer "F.Cu") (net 4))
 (segment (start 121.92 88.9) (end 123 88.9) (width 0.25) (layer "F.Cu") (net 4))
 (segment (start 125.575 103.775) (end 125.9 104.1) (width 0.25) (layer "F.Cu") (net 4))
 (segment (start 123.5 88.4) (end 123.7 88.2) (width 0.25) (layer "F.Cu") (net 4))
 (segment (start 138 105.1) (end 138 104.1) (width 0.25) (layer "F.Cu") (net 4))
 (segment (start 135.8 106.8716) (end 135.8 105.1) (width 0.25) (layer "F.Cu") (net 4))
 (segment (start 121.3612 87.7824) (end 123.2824 87.7824) (width 0.25) (layer "F.Cu") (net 4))
 (segment (start 119.85 96.6) (end 120.85 96.6) (width 0.25) (layer "F.Cu") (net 4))
 (segment (start 122.2088 80.534) (end 120.4976 82.2452) (width 0.25) (layer "F.Cu") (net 4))
 (segment (start 125.9 105.1) (end 125.9 106.1) (width 0.25) (layer "F.Cu") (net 4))
 (segment (start 128.3716 87.9284) (end 128.1 88.2) (width 0.25) (layer "F.Cu") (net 4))
 (segment (start 123.5 91.45) (end 123.5 88.4) (width 0.25) (layer "F.Cu") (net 4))
 (segment (start 133.275 89.525) (end 133.6 89.2) (width 0.25) (layer "F.Cu") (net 4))
 (segment (start 133.6 89.2) (end 133.6 88.2) (width 0.25) (layer "F.Cu") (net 4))
 (segment (start 120.4976 82.2452) (end 120.4976 86.9188) (width 0.25) (layer "F.Cu") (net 4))
 (segment (start 123 88.9) (end 123.7 88.2) (width 0.25) (layer "F.Cu") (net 4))
 (segment (start 138 105.1) (end 142.24 105.1) (width 0.25) (layer "F.Cu") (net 4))
 (segment (start 128.1 88.2) (end 128.1 89.2) (width 0.25) (layer "F.Cu") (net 4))
 (segment (start 121.92 95.53) (end 121.92 88.9) (width 0.25) (layer "F.Cu") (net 4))
 (segment (start 142.24 105.1) (end 144.76 105.1) (width 0.25) (layer "F.Cu") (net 4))
 (segment (start 120.85 96.6) (end 121.92 95.53) (width 0.25) (layer "F.Cu") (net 4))
 (segment (start 125.9 104.1) (end 125.9 105.1) (width 0.25) (layer "F.Cu") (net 4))
 (segment (start 123.7 89.2) (end 123.7 88.2) (width 0.25) (layer "F.Cu") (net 4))
 (segment (start 136.125 103.775) (end 135.8 104.1) (width 0.25) (layer "F.Cu") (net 4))
 (segment (start 124.025 103.775) (end 125.575 103.775) (width 0.25) (layer "F.Cu") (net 4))
 (segment (start 125.9 106.1) (end 126.7848 106.9848) (width 0.25) (layer "F.Cu") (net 4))
 (segment (start 132.5372 86.7156) (end 131.4196 86.7156) (width 0.25) (layer "F.Cu") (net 2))
 (segment (start 144.84 84.7) (end 144.84 82.1344) (width 0.25) (layer "F.Cu") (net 2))
 (segment (start 129.8956 108.1532) (end 131.826 108.1532) (width 0.25) (layer "F.Cu") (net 2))
 (segment (start 129.8956 109.0628) (end 129.8956 108.1532) (width 0.25) (layer "F.Cu") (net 2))
 (segment (start 131.4 86.7352) (end 131.4 88.2) (width 0.25) (layer "F.Cu") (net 2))
 (segment (start 144.84 84.7) (end 146.0844 84.7) (width 0.25) (layer "F.Cu") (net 2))
 (segment (start 131.4196 86.7156) (end 131.4 86.7352) (width 0.25) (layer "F.Cu") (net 2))
 (segment (start 132.0292 109.0628) (end 132.0292 107.95) (width 0.25) (layer "F.Cu") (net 2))
 (segment (start 131.826 108.1532) (end 132.0292 107.95) (width 0.25) (layer "F.Cu") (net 2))
 (segment (start 132.5372 88.1628) (end 132.5 88.2) (width 0.25) (layer "F.Cu") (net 2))
 (segment (start 146.0844 84.7) (end 146.4564 84.328) (width 0.25) (layer "F.Cu") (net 2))
 (segment (start 132.5372 86.7156) (end 132.5372 88.1628) (width 0.25) (layer "F.Cu") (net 2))
 (segment (start 146.4564 84.328) (end 146.4564 78.1304) (width 0.25) (layer "F.Cu") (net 2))
 (segment (start 144.84 82.1344) (end 144.8816 82.0928) (width 0.25) (layer "F.Cu") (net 2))
 (segment (start 123.9646 84.1122) (end 122.7836 85.2932) (width 0.25) (layer "F.Cu") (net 2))
 (segment (start 123.9646 82.4484) (end 123.9646 84.1122) (width 0.25) (layer "F.Cu") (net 2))
 (via (at 144.8816 82.0928) (size 0.8) (drill 0.4) (layers "F.Cu" "B.Cu") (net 2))
 (via (at 122.7836 85.2932) (size 0.8) (drill 0.4) (layers "F.Cu" "B.Cu") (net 2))
 (via (at 146.4564 78.1304) (size 0.8) (drill 0.4) (layers "F.Cu" "B.Cu") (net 2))
 (via (at 132.0292 107.95) (size 0.8) (drill 0.4) (layers "F.Cu" "B.Cu") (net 2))
 (via (at 132.5372 86.7156) (size 0.8) (drill 0.4) (layers "F.Cu" "B.Cu") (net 2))
 (segment (start 125.0696 78.1304) (end 121.7168 81.4832) (width 0.25) (layer "B.Cu") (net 2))
 (segment (start 138.7348 107.95) (end 139.5984 107.0864) (width 0.25) (layer "B.Cu") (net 2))
 (segment (start 132.0292 107.95) (end 138.7348 107.95) (width 0.25) (layer "B.Cu") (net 2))
 (segment (start 121.7168 85.1408) (end 121.666 85.1916) (width 0.25) (layer "B.Cu") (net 2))
 (segment (start 121.7168 81.4832) (end 121.7168 85.1408) (width 0.25) (layer "B.Cu") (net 2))
 (segment (start 121.666 85.1916) (end 122.682 85.1916) (width 0.25) (layer "B.Cu") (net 2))
 (segment (start 137.16 82.0928) (end 132.5372 86.7156) (width 0.25) (layer "B.Cu") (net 2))
 (segment (start 139.5984 107.0864) (end 139.5984 89.9416) (width 0.25) (layer "B.Cu") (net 2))
 (segment (start 139.5984 89.9416) (end 144.84 84.7) (width 0.25) (layer "B.Cu") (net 2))
 (segment (start 122.682 85.1916) (end 122.7836 85.2932) (width 0.25) (layer "B.Cu") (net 2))
 (segment (start 146.4564 78.1304) (end 125.0696 78.1304) (width 0.25) (layer "B.Cu") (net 2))
 (segment (start 144.8816 82.0928) (end 137.16 82.0928) (width 0.25) (layer "B.Cu") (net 2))
 (segment (start 130.3 105.1) (end 130.3 103.38) (width 0.25) (layer "F.Cu") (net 5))
 (segment (start 130.3 103.38) (end 130.3528 103.3272) (width 0.25) (layer "F.Cu") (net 5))
 (via (at 130.3528 103.3272) (size 0.8) (drill 0.4) (layers "F.Cu" "B.Cu") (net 5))
 (segment (start 117.7072 103.3272) (end 116.84 102.46) (width 0.25) (layer "B.Cu") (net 5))
 (segment (start 130.3528 103.3272) (end 117.7072 103.3272) (width 0.25) (layer "B.Cu") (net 5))
 (segment (start 119.85 102.1) (end 119.02 102.1) (width 0.25) (layer "F.Cu") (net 18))
 (segment (start 119.02 102.1) (end 116.84 99.92) (width 0.25) (layer "F.Cu") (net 18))
 (segment (start 118.85 99.9) (end 116.84 97.89) (width 0.25) (layer "F.Cu") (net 17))
 (segment (start 119.85 99.9) (end 118.85 99.9) (width 0.25) (layer "F.Cu") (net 17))
 (segment (start 116.84 97.89) (end 116.84 97.38) (width 0.25) (layer "F.Cu") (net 17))
 (segment (start 118.015 96.015) (end 116.84 94.84) (width 0.25) (layer "F.Cu") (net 16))
 (segment (start 118.015 97.965) (end 118.015 96.015) (width 0.25) (layer "F.Cu") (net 16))
 (segment (start 119.85 98.8) (end 118.85 98.8) (width 0.25) (layer "F.Cu") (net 16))
 (segment (start 118.85 98.8) (end 118.015 97.965) (width 0.25) (layer "F.Cu") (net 16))
 (segment (start 119.85 97.7) (end 118.85 97.7) (width 0.25) (layer "F.Cu") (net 15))
 (segment (start 118.85 97.7) (end 118.465 97.315) (width 0.25) (layer "F.Cu") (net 15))
 (segment (start 118.465 93.925) (end 116.84 92.3) (width 0.25) (layer "F.Cu") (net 15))
 (segment (start 118.465 97.315) (end 118.465 93.925) (width 0.25) (layer "F.Cu") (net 15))
 (segment (start 119.85 91.1) (end 118.18 91.1) (width 0.25) (layer "F.Cu") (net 14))
 (segment (start 118.18 91.1) (end 116.84 89.76) (width 0.25) (layer "F.Cu") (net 14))
 (segment (start 119.85 90) (end 117.07 87.22) (width 0.25) (layer "F.Cu") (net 13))
 (segment (start 117.07 87.22) (end 116.84 87.22) (width 0.25) (layer "F.Cu") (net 13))
 (segment (start 141.85 90) (end 144.61 87.24) (width 0.25) (layer "F.Cu") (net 11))
 (segment (start 144.61 87.24) (end 144.84 87.24) (width 0.25) (layer "F.Cu") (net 11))
 (segment (start 143.52 91.1) (end 144.84 89.78) (width 0.25) (layer "F.Cu") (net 10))
 (segment (start 141.85 91.1) (end 143.52 91.1) (width 0.25) (layer "F.Cu") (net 10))
 (segment (start 140.335 97.7) (end 140.3234 97.6884) (width 0.25) (layer "F.Cu") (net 9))
 (segment (start 141.85 97.7) (end 140.335 97.7) (width 0.25) (layer "F.Cu") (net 9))
 (via (at 140.3234 97.6884) (size 0.8) (drill 0.4) (layers "F.Cu" "B.Cu") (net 9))
 (segment (start 140.3234 97.6884) (end 140.3234 96.8366) (width 0.25) (layer "B.Cu") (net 9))
 (segment (start 140.3234 96.8366) (end 144.84 92.32) (width 0.25) (layer "B.Cu") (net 9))
 (segment (start 143.215 99.535) (end 143.215 96.485) (width 0.25) (layer "F.Cu") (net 8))
 (segment (start 143.215 96.485) (end 144.84 94.86) (width 0.25) (layer "F.Cu") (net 8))
 (segment (start 142.85 99.9) (end 143.215 99.535) (width 0.25) (layer "F.Cu") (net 8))
 (segment (start 141.85 99.9) (end 142.85 99.9) (width 0.25) (layer "F.Cu") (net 8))
 (segment (start 141.85 101) (end 143.091701 101) (width 0.25) (layer "F.Cu") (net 7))
 (segment (start 143.091701 101) (end 143.665 100.426701) (width 0.25) (layer "F.Cu") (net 7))
 (segment (start 143.665 100.426701) (end 143.665 98.575) (width 0.25) (layer "F.Cu") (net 7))
 (segment (start 143.665 98.575) (end 144.84 97.4) (width 0.25) (layer "F.Cu") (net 7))
 (segment (start 142.68 102.1) (end 144.84 99.94) (width 0.25) (layer "F.Cu") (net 6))
 (segment (start 141.85 102.1) (end 142.68 102.1) (width 0.25) (layer "F.Cu") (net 6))
 (segment (start 116.94 105.1) (end 116.84 105) (width 0.25) (layer "F.Cu") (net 21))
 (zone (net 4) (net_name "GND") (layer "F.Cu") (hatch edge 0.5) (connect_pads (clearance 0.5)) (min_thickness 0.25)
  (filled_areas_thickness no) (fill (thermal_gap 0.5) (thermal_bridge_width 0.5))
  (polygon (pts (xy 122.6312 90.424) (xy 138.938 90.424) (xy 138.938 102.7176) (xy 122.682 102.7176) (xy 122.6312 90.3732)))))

